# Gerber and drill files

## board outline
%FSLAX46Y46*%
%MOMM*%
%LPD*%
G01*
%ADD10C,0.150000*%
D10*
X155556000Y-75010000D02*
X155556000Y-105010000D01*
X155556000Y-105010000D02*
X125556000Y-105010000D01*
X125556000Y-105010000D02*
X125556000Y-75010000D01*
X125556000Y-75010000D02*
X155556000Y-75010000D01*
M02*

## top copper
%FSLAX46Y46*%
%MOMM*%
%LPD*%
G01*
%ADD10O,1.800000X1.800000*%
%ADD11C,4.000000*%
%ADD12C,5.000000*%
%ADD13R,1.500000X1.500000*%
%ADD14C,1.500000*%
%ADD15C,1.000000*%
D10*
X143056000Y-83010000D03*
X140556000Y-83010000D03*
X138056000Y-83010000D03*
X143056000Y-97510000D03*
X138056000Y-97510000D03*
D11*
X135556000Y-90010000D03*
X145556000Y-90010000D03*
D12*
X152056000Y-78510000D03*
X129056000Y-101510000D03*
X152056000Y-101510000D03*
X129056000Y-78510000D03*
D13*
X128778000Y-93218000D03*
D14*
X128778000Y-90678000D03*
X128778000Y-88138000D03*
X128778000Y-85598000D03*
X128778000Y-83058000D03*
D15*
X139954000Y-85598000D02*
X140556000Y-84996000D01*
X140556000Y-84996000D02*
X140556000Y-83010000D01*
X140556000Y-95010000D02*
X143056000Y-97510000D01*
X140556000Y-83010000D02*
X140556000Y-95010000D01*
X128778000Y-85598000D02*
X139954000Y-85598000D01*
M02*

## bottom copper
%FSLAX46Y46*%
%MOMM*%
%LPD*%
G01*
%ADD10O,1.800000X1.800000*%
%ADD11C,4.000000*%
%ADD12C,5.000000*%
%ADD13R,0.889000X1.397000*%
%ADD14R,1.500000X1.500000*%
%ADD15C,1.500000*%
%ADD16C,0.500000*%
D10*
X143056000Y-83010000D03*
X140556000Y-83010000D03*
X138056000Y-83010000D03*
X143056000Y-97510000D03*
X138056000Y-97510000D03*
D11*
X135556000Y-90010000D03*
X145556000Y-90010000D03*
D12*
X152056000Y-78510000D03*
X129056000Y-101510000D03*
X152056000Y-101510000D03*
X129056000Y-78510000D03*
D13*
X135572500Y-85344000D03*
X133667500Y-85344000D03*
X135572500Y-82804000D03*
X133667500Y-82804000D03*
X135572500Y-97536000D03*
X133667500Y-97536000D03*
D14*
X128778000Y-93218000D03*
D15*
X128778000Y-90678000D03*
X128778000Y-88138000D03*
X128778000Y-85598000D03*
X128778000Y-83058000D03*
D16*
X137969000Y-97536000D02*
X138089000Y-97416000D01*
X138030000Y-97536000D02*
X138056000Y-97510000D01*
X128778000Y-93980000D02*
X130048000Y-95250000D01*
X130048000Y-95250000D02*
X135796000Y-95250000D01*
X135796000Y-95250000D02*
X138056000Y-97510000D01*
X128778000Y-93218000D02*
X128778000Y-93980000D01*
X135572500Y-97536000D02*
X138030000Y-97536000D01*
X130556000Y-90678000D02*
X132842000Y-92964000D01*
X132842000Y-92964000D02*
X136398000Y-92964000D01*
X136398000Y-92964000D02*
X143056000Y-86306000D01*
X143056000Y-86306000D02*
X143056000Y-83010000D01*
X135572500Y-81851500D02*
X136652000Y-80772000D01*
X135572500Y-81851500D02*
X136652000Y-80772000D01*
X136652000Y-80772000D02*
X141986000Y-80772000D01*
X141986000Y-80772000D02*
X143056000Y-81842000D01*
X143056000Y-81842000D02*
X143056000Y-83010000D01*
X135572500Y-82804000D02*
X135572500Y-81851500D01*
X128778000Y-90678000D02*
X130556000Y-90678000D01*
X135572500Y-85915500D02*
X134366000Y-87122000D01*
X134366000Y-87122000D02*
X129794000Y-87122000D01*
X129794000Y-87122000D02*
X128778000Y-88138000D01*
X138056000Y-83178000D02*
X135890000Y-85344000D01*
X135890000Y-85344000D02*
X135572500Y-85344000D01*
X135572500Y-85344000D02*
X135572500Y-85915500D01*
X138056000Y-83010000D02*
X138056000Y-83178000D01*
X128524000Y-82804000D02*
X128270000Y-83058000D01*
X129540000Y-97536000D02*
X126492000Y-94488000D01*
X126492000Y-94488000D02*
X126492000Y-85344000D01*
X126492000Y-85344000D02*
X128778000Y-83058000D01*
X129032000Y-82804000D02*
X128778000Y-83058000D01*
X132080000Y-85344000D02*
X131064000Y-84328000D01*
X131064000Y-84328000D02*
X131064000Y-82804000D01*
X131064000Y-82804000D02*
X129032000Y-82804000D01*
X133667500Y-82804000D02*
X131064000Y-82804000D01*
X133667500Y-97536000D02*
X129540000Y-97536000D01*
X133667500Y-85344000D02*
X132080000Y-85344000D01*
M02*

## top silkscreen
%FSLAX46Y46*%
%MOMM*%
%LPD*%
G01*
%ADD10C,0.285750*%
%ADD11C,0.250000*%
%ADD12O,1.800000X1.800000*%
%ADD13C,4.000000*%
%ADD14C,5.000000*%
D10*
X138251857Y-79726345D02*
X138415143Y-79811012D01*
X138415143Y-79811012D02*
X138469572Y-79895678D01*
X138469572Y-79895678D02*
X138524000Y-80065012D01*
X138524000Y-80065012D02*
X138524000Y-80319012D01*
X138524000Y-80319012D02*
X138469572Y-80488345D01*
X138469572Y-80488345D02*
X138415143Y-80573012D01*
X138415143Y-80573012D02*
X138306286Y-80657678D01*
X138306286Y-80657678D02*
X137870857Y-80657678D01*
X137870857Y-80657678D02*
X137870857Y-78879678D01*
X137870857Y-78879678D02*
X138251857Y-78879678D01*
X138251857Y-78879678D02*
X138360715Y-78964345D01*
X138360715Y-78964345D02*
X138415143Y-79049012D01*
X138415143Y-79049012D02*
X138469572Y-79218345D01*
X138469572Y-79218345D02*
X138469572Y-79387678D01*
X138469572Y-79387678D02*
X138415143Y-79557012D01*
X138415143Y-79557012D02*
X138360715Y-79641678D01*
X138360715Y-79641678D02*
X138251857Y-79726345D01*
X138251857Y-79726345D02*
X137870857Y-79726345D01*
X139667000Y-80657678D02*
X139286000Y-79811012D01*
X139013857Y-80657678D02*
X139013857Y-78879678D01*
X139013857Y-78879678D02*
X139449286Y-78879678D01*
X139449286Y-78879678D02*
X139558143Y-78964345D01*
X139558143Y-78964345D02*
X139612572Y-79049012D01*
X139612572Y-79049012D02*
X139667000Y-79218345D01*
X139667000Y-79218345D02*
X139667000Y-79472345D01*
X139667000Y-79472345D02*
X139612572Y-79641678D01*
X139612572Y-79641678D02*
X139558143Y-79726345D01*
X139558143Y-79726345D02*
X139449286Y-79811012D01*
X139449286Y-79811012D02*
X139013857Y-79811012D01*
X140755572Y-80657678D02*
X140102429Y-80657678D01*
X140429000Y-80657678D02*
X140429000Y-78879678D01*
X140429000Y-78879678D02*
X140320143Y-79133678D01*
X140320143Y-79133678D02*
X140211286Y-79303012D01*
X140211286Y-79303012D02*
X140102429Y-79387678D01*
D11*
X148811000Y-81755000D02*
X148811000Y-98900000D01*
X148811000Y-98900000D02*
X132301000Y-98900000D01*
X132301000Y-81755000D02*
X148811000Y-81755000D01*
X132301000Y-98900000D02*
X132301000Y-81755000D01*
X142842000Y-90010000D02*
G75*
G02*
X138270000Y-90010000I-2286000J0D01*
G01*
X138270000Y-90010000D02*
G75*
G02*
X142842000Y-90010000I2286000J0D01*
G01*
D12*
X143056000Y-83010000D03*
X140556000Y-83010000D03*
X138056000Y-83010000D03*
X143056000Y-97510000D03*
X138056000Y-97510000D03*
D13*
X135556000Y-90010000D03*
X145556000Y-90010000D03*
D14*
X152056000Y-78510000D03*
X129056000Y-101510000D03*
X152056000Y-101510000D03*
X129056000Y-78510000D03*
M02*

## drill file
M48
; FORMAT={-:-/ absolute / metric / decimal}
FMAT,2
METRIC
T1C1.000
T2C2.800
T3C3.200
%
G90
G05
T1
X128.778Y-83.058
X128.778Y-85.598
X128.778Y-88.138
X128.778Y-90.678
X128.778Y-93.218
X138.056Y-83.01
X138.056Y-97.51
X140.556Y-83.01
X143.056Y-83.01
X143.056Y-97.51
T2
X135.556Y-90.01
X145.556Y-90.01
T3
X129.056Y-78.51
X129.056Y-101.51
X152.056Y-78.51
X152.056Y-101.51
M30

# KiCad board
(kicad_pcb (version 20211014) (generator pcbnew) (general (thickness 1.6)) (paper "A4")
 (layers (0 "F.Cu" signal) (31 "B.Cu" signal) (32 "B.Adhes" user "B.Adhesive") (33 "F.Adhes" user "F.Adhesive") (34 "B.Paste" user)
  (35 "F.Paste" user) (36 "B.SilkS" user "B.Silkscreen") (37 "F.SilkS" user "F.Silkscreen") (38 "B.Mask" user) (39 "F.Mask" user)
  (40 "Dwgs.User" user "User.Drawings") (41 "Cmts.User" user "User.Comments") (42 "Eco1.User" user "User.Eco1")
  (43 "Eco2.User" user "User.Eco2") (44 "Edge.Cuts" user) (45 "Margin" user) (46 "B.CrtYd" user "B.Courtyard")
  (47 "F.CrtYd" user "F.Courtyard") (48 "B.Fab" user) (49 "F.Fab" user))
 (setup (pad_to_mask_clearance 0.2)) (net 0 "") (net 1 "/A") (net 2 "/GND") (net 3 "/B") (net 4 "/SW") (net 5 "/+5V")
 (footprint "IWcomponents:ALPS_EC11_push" (layer "F.Cu") (at 140.556 90.01)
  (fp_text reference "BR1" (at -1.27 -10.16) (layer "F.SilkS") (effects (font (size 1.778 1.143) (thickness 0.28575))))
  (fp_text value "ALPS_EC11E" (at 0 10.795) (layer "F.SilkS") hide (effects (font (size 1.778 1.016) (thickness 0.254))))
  (fp_line (start 8.255 -8.255) (end 8.255 8.89) (layer "F.SilkS") (width 0.25))
  (fp_line (start 8.255 8.89) (end -8.255 8.89) (layer "F.SilkS") (width 0.25))
  (fp_line (start -8.255 -8.255) (end 8.255 -8.255) (layer "F.SilkS") (width 0.25))
  (fp_line (start -8.255 8.89) (end -8.255 -8.255) (layer "F.SilkS") (width 0.25))
  (fp_circle (center 0 0) (end 2.286 0) (layer "F.SilkS") (width 0.25) (fill none))
  (pad "1" thru_hole oval locked (at 2.5 -7) (size 1.8 1.8) (drill 1) (layers *.Cu *.Mask "F.SilkS") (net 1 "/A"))
  (pad "2" thru_hole oval locked (at 0 -7) (size 1.8 1.8) (drill 1) (layers *.Cu *.Mask "F.SilkS") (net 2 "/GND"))
  (pad "3" thru_hole oval locked (at -2.5 -7) (size 1.8 1.8) (drill 1) (layers *.Cu *.Mask "F.SilkS") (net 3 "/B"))
  (pad "4" thru_hole oval locked (at 2.5 7.5) (size 1.8 1.8) (drill 1) (layers *.Cu *.Mask "F.SilkS") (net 2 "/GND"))
  (pad "5" thru_hole oval locked (at -2.5 7.5) (size 1.8 1.8) (drill 1) (layers *.Cu *.Mask "F.SilkS") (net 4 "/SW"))
  (pad "6" thru_hole circle locked (at -5 0) (size 4 4) (drill 2.8) (layers *.Cu *.Mask "F.SilkS"))
  (pad "7" thru_hole circle locked (at 5 0) (size 4 4) (drill 2.8) (layers *.Cu *.Mask "F.SilkS")))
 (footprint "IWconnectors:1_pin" (layer "F.Cu") (at 151.384 80.518)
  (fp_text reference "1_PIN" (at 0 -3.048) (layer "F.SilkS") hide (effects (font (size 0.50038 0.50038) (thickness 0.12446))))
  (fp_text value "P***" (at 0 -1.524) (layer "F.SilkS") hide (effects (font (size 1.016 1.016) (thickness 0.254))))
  (pad "1" thru_hole circle locked (at 0.672 -2.008) (size 5 5) (drill 3.2) (layers *.Cu *.Mask "F.SilkS")))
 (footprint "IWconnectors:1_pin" (layer "F.Cu") (at 130.556 100.076)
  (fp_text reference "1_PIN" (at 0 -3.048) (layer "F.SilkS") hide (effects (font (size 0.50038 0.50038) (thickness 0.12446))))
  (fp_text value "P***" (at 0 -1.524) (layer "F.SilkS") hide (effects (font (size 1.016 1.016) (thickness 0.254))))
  (pad "1" thru_hole circle locked (at -1.5 1.434) (size 5 5) (drill 3.2) (layers *.Cu *.Mask "F.SilkS")))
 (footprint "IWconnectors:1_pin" (layer "F.Cu") (at 152.4 101.854)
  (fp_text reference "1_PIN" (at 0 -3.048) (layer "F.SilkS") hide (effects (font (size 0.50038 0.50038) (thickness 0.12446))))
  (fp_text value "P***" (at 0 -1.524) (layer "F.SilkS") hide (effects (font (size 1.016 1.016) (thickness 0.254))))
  (pad "1" thru_hole circle locked (at -0.344 -0.344) (size 5 5) (drill 3.2) (layers *.Cu *.Mask "F.SilkS")))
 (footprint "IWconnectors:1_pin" (layer "F.Cu") (at 130.556 80.01)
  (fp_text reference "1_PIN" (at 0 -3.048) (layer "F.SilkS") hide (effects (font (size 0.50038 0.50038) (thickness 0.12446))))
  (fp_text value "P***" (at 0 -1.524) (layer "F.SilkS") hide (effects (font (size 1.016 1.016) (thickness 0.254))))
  (pad "1" thru_hole circle locked (at -1.5 -1.5) (size 5 5) (drill 3.2) (layers *.Cu *.Mask "F.SilkS")))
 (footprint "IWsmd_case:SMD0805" (layer "B.Cu") (at 134.62 85.344 180)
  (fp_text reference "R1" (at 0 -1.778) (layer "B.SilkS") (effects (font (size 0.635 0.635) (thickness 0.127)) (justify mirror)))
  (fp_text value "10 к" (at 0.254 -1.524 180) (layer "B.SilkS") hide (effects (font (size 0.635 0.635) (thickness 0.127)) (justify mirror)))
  (pad "1" smd rect locked (at -0.9525 0 180) (size 0.889 1.397) (layers "B.Cu" "B.Paste" "B.Mask") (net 3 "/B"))
  (pad "2" smd rect locked (at 0.9525 0 180) (size 0.889 1.397) (layers "B.Cu" "B.Paste" "B.Mask") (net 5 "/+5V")))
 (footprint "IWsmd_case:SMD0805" (layer "B.Cu") (at 134.62 82.804 180)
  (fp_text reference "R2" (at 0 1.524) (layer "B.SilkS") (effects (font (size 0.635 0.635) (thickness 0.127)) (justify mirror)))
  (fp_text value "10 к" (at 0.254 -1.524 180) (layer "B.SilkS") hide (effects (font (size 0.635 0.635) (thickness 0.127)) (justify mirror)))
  (pad "1" smd rect locked (at -0.9525 0 180) (size 0.889 1.397) (layers "B.Cu" "B.Paste" "B.Mask") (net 1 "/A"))
  (pad "2" smd rect locked (at 0.9525 0 180) (size 0.889 1.397) (layers "B.Cu" "B.Paste" "B.Mask") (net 5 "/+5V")))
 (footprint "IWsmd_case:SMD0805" (layer "B.Cu") (at 134.62 97.536 180)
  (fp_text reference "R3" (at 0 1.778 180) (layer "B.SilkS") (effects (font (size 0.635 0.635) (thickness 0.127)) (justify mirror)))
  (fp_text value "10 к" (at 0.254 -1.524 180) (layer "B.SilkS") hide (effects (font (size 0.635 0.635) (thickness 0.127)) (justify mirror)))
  (pad "1" smd rect locked (at -0.9525 0 180) (size 0.889 1.397) (layers "B.Cu" "B.Paste" "B.Mask") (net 4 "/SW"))
  (pad "2" smd rect locked (at 0.9525 0 180) (size 0.889 1.397) (layers "B.Cu" "B.Paste" "B.Mask") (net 5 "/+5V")))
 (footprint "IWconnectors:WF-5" (layer "B.Cu") (at 128.778 88.138 90)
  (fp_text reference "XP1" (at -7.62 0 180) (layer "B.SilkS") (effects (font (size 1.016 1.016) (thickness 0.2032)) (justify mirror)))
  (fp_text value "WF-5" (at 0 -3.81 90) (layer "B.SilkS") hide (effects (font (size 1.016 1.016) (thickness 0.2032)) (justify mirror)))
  (pad "1" thru_hole rect locked (at -5.08 0 90) (size 1.5 1.5) (drill 1) (layers *.Cu *.Mask "B.SilkS") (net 4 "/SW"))
  (pad "2" thru_hole circle locked (at -2.54 0 90) (size 1.5 1.5) (drill 1) (layers *.Cu *.Mask "B.SilkS") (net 1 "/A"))
  (pad "3" thru_hole circle locked (at 0 0 90) (size 1.5 1.5) (drill 1) (layers *.Cu *.Mask "B.SilkS") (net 3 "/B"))
  (pad "4" thru_hole circle locked (at 2.54 0 90) (size 1.5 1.5) (drill 1) (layers *.Cu *.Mask "B.SilkS") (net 2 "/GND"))
  (pad "5" thru_hole circle locked (at 5.08 0 90) (size 1.5 1.5) (drill 1) (layers *.Cu *.Mask "B.SilkS") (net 5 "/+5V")))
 (gr_line (start 155.556 75.01) (end 155.556 105.01) (layer "Edge.Cuts") (width 0.15))
 (gr_line (start 155.556 105.01) (end 125.556 105.01) (layer "Edge.Cuts") (width 0.15))
 (gr_line (start 125.556 105.01) (end 125.556 75.01) (layer "Edge.Cuts") (width 0.15))
 (gr_line (start 125.556 75.01) (end 155.556 75.01) (layer "Edge.Cuts") (width 0.15))
 (segment (start 137.969 97.536) (end 138.089 97.416) (width 0.5) (layer "B.Cu") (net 4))
 (segment (start 138.03 97.536) (end 138.056 97.51) (width 0.5) (layer "B.Cu") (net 4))
 (segment (start 128.778 93.98) (end 130.048 95.25) (width 0.5) (layer "B.Cu") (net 4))
 (segment (start 130.048 95.25) (end 135.796 95.25) (width 0.5) (layer "B.Cu") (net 4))
 (segment (start 135.796 95.25) (end 138.056 97.51) (width 0.5) (layer "B.Cu") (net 4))
 (segment (start 128.778 93.218) (end 128.778 93.98) (width 0.5) (layer "B.Cu") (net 4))
 (segment (start 135.5725 97.536) (end 138.03 97.536) (width 0.5) (layer "B.Cu") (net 4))
 (segment (start 139.954 85.598) (end 140.556 84.996) (width 1) (layer "F.Cu") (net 2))
 (segment (start 140.556 84.996) (end 140.556 83.01) (width 1) (layer "F.Cu") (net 2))
 (segment (start 140.556 95.01) (end 143.056 97.51) (width 1) (layer "F.Cu") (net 2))
 (segment (start 140.556 83.01) (end 140.556 95.01) (width 1) (layer "F.Cu") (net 2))
 (segment (start 128.778 85.598) (end 139.954 85.598) (width 1) (layer "F.Cu") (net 2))
 (segment (start 130.556 90.678) (end 132.842 92.964) (width 0.5) (layer "B.Cu") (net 1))
 (segment (start 132.842 92.964) (end 136.398 92.964) (width 0.5) (layer "B.Cu") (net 1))
 (segment (start 136.398 92.964) (end 143.056 86.306) (width 0.5) (layer "B.Cu") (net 1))
 (segment (start 143.056 86.306) (end 143.056 83.01) (width 0.5) (layer "B.Cu") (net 1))
 (segment (start 135.5725 81.8515) (end 136.652 80.772) (width 0.5) (layer "B.Cu") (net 1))
 (segment (start 135.5725 81.8515) (end 136.652 80.772) (width 0.5) (layer "B.Cu") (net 1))
 (segment (start 136.652 80.772) (end 141.986 80.772) (width 0.5) (layer "B.Cu") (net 1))
 (segment (start 141.986 80.772) (end 143.056 81.842) (width 0.5) (layer "B.Cu") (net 1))
 (segment (start 143.056 81.842) (end 143.056 83.01) (width 0.5) (layer "B.Cu") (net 1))
 (segment (start 135.5725 82.804) (end 135.5725 81.8515) (width 0.5) (layer "B.Cu") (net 1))
 (segment (start 128.778 90.678) (end 130.556 90.678) (width 0.5) (layer "B.Cu") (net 1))
 (segment (start 135.5725 85.9155) (end 134.366 87.122) (width 0.5) (layer "B.Cu") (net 3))
 (segment (start 134.366 87.122) (end 129.794 87.122) (width 0.5) (layer "B.Cu") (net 3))
 (segment (start 129.794 87.122) (end 128.778 88.138) (width 0.5) (layer "B.Cu") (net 3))
 (segment (start 138.056 83.178) (end 135.89 85.344) (width 0.5) (layer "B.Cu") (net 3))
 (segment (start 135.89 85.344) (end 135.5725 85.344) (width 0.5) (layer "B.Cu") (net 3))
 (segment (start 135.5725 85.344) (end 135.5725 85.9155) (width 0.5) (layer "B.Cu") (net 3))
 (segment (start 138.056 83.01) (end 138.056 83.178) (width 0.5) (layer "B.Cu") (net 3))
 (segment (start 128.524 82.804) (end 128.27 83.058) (width 0.5) (layer "B.Cu") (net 5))
 (segment (start 129.54 97.536) (end 126.492 94.488) (width 0.5) (layer "B.Cu") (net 5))
 (segment (start 126.492 94.488) (end 126.492 85.344) (width 0.5) (layer "B.Cu") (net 5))
 (segment (start 126.492 85.344) (end 128.778 83.058) (width 0.5) (layer "B.Cu") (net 5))
 (segment (start 129.032 82.804) (end 128.778 83.058) (width 0.5) (layer "B.Cu") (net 5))
 (segment (start 132.08 85.344) (end 131.064 84.328) (width 0.5) (layer "B.Cu") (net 5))
 (segment (start 131.064 84.328) (end 131.064 82.804) (width 0.5) (layer "B.Cu") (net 5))
 (segment (start 131.064 82.804) (end 129.032 82.804) (width 0.5) (layer "B.Cu") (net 5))
 (segment (start 133.6675 82.804) (end 131.064 82.804) (width 0.5) (layer "B.Cu") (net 5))
 (segment (start 133.6675 97.536) (end 129.54 97.536) (width 0.5) (layer "B.Cu") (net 5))
 (segment (start 133.6675 85.344) (end 132.08 85.344) (width 0.5) (layer "B.Cu") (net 5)))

